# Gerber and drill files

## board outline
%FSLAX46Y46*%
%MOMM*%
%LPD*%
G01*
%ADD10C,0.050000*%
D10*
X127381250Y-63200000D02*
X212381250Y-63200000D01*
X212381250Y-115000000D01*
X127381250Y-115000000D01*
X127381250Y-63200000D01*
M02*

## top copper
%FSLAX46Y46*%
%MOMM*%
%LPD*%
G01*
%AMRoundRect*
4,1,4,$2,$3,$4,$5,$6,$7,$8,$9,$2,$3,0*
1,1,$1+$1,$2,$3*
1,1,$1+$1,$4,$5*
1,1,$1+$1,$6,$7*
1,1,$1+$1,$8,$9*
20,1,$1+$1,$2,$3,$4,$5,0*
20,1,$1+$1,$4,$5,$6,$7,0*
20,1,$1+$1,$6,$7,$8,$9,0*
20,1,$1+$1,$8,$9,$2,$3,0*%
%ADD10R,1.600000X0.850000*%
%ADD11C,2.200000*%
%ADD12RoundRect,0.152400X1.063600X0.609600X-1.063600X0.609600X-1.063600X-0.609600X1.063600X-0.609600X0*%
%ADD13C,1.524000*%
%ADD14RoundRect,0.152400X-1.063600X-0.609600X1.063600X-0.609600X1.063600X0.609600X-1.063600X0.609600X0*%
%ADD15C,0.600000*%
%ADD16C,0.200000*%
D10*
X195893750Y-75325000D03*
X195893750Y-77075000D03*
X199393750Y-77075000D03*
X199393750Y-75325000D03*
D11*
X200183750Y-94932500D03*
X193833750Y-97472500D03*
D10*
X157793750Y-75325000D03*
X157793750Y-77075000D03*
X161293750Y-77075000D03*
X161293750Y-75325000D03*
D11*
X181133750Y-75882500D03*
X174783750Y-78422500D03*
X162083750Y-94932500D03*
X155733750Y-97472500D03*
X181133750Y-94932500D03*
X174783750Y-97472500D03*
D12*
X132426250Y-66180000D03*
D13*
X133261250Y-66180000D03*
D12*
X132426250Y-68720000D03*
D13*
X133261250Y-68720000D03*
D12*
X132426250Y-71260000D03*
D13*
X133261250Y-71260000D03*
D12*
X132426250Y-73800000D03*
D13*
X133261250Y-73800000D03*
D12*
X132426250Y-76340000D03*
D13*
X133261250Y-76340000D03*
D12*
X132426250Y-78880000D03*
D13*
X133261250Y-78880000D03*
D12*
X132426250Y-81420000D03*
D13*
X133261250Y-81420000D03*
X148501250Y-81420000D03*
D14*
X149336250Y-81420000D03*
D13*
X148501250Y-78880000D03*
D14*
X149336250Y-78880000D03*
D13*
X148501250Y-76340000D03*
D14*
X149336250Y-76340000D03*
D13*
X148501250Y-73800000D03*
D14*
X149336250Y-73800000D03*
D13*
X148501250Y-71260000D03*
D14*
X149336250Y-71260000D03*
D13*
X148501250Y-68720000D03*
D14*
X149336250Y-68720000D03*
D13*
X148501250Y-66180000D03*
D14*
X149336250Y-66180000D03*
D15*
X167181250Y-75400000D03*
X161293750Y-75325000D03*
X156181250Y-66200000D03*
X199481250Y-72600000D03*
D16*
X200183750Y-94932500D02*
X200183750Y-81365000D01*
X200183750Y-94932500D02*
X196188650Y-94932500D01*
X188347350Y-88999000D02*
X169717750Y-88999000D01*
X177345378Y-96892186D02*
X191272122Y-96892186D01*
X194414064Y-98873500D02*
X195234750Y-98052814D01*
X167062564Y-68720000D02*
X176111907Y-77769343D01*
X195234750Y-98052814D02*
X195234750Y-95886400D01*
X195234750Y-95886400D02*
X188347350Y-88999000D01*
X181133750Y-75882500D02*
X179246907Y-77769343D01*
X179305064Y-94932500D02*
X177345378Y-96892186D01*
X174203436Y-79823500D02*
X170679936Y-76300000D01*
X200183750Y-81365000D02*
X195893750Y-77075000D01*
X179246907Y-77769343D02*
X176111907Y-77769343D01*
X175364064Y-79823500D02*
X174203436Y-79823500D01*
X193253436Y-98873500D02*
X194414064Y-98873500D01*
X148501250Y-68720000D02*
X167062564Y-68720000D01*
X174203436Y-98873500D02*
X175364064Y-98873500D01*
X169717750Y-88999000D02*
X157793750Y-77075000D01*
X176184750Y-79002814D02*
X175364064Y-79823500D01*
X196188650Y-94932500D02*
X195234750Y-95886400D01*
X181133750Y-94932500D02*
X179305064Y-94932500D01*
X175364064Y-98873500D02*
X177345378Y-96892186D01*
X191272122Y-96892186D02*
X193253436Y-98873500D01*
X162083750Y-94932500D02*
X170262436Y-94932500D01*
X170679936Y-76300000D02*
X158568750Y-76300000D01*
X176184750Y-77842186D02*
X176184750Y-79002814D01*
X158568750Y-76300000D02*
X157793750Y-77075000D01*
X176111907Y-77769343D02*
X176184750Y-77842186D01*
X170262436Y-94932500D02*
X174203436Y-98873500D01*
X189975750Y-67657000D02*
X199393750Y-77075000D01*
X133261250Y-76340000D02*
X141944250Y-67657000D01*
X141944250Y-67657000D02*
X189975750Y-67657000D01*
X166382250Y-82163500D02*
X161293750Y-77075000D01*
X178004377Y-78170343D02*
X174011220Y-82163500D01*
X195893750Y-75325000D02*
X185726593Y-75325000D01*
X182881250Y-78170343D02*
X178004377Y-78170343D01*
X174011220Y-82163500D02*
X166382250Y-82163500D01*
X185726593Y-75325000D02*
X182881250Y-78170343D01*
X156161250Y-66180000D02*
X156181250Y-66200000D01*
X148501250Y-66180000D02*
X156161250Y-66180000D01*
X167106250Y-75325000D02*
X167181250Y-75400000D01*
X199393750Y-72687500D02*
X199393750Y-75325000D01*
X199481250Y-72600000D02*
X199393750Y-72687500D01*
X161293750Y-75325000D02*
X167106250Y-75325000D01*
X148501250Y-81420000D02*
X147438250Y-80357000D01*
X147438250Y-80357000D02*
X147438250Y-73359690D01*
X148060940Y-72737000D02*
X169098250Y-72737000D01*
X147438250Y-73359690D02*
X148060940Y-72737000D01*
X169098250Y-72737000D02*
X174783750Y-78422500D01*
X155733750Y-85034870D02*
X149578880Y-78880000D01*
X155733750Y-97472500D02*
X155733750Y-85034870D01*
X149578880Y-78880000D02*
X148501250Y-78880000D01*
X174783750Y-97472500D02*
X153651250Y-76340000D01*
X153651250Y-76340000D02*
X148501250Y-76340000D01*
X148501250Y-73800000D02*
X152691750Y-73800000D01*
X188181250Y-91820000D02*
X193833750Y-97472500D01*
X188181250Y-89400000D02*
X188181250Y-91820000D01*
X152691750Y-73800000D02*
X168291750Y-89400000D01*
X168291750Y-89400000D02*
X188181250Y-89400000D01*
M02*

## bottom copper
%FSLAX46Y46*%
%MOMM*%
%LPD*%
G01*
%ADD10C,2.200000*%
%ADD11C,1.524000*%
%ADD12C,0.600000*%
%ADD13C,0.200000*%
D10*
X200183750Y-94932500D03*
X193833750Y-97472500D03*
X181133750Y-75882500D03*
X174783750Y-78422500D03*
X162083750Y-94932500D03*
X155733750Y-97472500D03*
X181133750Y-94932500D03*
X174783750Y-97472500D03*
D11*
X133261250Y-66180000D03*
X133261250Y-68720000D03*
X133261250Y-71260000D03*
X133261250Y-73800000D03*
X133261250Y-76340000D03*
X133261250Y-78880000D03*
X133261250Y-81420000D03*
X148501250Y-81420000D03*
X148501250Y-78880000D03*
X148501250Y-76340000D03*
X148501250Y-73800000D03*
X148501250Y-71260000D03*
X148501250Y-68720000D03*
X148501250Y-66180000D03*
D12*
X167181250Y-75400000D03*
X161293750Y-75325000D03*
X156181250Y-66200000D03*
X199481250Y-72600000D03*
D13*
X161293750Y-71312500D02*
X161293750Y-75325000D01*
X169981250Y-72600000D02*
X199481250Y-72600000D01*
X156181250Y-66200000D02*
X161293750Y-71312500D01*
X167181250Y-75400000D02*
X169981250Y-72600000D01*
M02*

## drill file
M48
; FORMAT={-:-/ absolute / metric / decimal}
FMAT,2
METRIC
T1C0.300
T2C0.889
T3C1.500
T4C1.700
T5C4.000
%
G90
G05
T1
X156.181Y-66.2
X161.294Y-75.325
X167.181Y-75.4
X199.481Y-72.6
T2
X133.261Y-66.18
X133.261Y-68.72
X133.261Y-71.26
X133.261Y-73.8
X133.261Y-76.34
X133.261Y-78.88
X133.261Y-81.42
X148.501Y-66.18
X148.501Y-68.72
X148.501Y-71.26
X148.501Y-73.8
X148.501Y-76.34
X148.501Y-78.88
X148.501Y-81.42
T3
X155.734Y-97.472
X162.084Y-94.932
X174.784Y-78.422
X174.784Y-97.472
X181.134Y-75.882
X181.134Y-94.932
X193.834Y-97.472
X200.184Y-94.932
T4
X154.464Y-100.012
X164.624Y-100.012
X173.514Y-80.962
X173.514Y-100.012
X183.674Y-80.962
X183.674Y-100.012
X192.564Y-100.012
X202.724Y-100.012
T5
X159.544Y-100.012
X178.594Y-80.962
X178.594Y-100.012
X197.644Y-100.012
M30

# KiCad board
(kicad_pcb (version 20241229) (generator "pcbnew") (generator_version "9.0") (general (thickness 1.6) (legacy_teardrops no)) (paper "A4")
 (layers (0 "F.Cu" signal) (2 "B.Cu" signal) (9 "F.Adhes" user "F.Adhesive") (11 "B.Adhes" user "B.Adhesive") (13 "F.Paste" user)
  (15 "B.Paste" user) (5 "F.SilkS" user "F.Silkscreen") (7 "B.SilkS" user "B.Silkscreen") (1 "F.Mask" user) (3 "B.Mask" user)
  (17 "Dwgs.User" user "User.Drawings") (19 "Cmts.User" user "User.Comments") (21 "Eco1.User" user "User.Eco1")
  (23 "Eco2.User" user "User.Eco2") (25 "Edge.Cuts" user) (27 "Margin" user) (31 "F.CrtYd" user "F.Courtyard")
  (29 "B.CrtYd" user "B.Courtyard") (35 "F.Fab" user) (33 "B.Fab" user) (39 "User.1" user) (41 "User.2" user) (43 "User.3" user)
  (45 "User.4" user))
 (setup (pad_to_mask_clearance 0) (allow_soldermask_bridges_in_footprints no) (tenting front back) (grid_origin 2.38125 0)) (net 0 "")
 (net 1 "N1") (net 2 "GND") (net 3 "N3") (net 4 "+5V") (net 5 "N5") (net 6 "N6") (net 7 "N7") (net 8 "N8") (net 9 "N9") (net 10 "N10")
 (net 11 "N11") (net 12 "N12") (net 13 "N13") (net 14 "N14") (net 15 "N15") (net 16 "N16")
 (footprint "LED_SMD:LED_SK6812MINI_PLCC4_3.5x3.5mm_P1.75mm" (layer "F.Cu") (at 197.64375 76.2)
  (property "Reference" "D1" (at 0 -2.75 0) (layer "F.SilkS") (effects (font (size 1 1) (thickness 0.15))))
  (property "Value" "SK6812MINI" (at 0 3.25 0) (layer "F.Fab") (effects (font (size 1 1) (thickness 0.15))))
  (pad "1" smd rect (at -1.75 -0.875) (size 1.6 0.85) (layers "F.Cu" "F.Mask" "F.Paste") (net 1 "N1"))
  (pad "2" smd rect (at -1.75 0.875) (size 1.6 0.85) (layers "F.Cu" "F.Mask" "F.Paste") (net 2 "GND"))
  (pad "3" smd rect (at 1.75 0.875) (size 1.6 0.85) (layers "F.Cu" "F.Mask" "F.Paste") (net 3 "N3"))
  (pad "4" smd rect (at 1.75 -0.875) (size 1.6 0.85) (layers "F.Cu" "F.Mask" "F.Paste") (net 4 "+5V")))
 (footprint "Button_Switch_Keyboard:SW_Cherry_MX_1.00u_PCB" (layer "F.Cu") (at 200.18375 94.9325)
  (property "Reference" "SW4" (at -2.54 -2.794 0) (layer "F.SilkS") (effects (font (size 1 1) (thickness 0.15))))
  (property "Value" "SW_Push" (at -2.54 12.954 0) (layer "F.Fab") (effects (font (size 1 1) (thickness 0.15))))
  (pad "" np_thru_hole circle (at -7.62 5.08) (size 1.7 1.7) (drill 1.7) (layers "*.Cu" "*.Mask"))
  (pad "" np_thru_hole circle (at -2.54 5.08) (size 4 4) (drill 4) (layers "*.Cu" "*.Mask"))
  (pad "" np_thru_hole circle (at 2.54 5.08) (size 1.7 1.7) (drill 1.7) (layers "*.Cu" "*.Mask"))
  (pad "1" thru_hole circle (at 0 0) (size 2.2 2.2) (drill 1.5) (layers "*.Cu" "*.Mask") (remove_unused_layers no) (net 2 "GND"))
  (pad "2" thru_hole circle (at -6.35 2.54) (size 2.2 2.2) (drill 1.5) (layers "*.Cu" "*.Mask") (remove_unused_layers no) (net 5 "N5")))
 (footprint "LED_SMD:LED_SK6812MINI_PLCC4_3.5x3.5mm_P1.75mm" (layer "F.Cu") (at 159.54375 76.2)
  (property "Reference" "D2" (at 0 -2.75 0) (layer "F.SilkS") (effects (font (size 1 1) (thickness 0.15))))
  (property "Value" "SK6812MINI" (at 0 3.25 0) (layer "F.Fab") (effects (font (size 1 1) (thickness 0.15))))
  (pad "1" smd rect (at -1.75 -0.875) (size 1.6 0.85) (layers "F.Cu" "F.Mask" "F.Paste") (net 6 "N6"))
  (pad "2" smd rect (at -1.75 0.875) (size 1.6 0.85) (layers "F.Cu" "F.Mask" "F.Paste") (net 2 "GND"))
  (pad "3" smd rect (at 1.75 0.875) (size 1.6 0.85) (layers "F.Cu" "F.Mask" "F.Paste") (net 1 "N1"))
  (pad "4" smd rect (at 1.75 -0.875) (size 1.6 0.85) (layers "F.Cu" "F.Mask" "F.Paste") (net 4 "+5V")))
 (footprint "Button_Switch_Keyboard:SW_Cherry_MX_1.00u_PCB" (layer "F.Cu") (at 181.13375 75.8825)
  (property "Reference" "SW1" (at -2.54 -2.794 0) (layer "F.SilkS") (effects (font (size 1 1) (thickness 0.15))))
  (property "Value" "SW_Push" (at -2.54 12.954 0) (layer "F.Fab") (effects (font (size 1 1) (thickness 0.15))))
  (pad "" np_thru_hole circle (at -7.62 5.08) (size 1.7 1.7) (drill 1.7) (layers "*.Cu" "*.Mask"))
  (pad "" np_thru_hole circle (at -2.54 5.08) (size 4 4) (drill 4) (layers "*.Cu" "*.Mask"))
  (pad "" np_thru_hole circle (at 2.54 5.08) (size 1.7 1.7) (drill 1.7) (layers "*.Cu" "*.Mask"))
  (pad "1" thru_hole circle (at 0 0) (size 2.2 2.2) (drill 1.5) (layers "*.Cu" "*.Mask") (remove_unused_layers no) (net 2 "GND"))
  (pad "2" thru_hole circle (at -6.35 2.54) (size 2.2 2.2) (drill 1.5) (layers "*.Cu" "*.Mask") (remove_unused_layers no) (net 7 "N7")))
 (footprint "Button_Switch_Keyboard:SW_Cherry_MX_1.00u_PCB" (layer "F.Cu") (at 162.08375 94.9325)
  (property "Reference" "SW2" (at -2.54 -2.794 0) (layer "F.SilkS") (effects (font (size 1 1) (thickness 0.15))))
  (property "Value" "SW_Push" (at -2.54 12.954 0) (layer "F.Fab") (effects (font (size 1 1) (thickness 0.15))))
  (pad "" np_thru_hole circle (at -7.62 5.08) (size 1.7 1.7) (drill 1.7) (layers "*.Cu" "*.Mask"))
  (pad "" np_thru_hole circle (at -2.54 5.08) (size 4 4) (drill 4) (layers "*.Cu" "*.Mask"))
  (pad "" np_thru_hole circle (at 2.54 5.08) (size 1.7 1.7) (drill 1.7) (layers "*.Cu" "*.Mask"))
  (pad "1" thru_hole circle (at 0 0) (size 2.2 2.2) (drill 1.5) (layers "*.Cu" "*.Mask") (remove_unused_layers no) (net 2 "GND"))
  (pad "2" thru_hole circle (at -6.35 2.54) (size 2.2 2.2) (drill 1.5) (layers "*.Cu" "*.Mask") (remove_unused_layers no) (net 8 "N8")))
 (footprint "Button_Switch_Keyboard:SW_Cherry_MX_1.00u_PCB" (layer "F.Cu") (at 181.13375 94.9325)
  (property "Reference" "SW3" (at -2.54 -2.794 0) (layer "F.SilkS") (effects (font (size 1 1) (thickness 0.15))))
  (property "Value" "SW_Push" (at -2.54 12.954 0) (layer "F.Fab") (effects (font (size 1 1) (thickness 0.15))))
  (pad "" np_thru_hole circle (at -7.62 5.08) (size 1.7 1.7) (drill 1.7) (layers "*.Cu" "*.Mask"))
  (pad "" np_thru_hole circle (at -2.54 5.08) (size 4 4) (drill 4) (layers "*.Cu" "*.Mask"))
  (pad "" np_thru_hole circle (at 2.54 5.08) (size 1.7 1.7) (drill 1.7) (layers "*.Cu" "*.Mask"))
  (pad "1" thru_hole circle (at 0 0) (size 2.2 2.2) (drill 1.5) (layers "*.Cu" "*.Mask") (remove_unused_layers no) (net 2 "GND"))
  (pad "2" thru_hole circle (at -6.35 2.54) (size 2.2 2.2) (drill 1.5) (layers "*.Cu" "*.Mask") (remove_unused_layers no) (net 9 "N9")))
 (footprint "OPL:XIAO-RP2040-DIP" (layer "F.Cu") (at 140.88125 73.8)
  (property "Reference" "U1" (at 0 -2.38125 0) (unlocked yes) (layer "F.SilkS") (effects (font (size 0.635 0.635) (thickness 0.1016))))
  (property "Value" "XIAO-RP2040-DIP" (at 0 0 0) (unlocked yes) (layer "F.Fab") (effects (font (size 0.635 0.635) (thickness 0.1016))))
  (pad "1" smd roundrect (at -8.455 -7.62 180) (size 2.432 1.524) (layers "F.Cu" "F.Mask") (roundrect_rratio 0.1) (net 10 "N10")
   (thermal_bridge_angle 45))
  (pad "1" thru_hole circle (at -7.62 -7.62 180) (size 1.524 1.524) (drill 0.889) (layers "*.Cu" "*.Mask") (remove_unused_layers no)
   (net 10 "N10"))
  (pad "2" smd roundrect (at -8.455 -5.08 180) (size 2.432 1.524) (layers "F.Cu" "F.Mask") (roundrect_rratio 0.1) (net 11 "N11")
   (thermal_bridge_angle 45))
  (pad "2" thru_hole circle (at -7.62 -5.08 180) (size 1.524 1.524) (drill 0.889) (layers "*.Cu" "*.Mask") (remove_unused_layers no)
   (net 11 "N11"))
  (pad "3" smd roundrect (at -8.455 -2.54 180) (size 2.432 1.524) (layers "F.Cu" "F.Mask") (roundrect_rratio 0.1) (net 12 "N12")
   (thermal_bridge_angle 45))
  (pad "3" thru_hole circle (at -7.62 -2.54 180) (size 1.524 1.524) (drill 0.889) (layers "*.Cu" "*.Mask") (remove_unused_layers no)
   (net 12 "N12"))
  (pad "4" smd roundrect (at -8.455 0 180) (size 2.432 1.524) (layers "F.Cu" "F.Mask") (roundrect_rratio 0.1) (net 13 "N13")
   (thermal_bridge_angle 45))
  (pad "4" thru_hole circle (at -7.62 0 180) (size 1.524 1.524) (drill 0.889) (layers "*.Cu" "*.Mask") (remove_unused_layers no)
   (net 13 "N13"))
  (pad "5" smd roundrect (at -8.455 2.54 180) (size 2.432 1.524) (layers "F.Cu" "F.Mask") (roundrect_rratio 0.1) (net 3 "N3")
   (thermal_bridge_angle 45))
  (pad "5" thru_hole circle (at -7.62 2.54 180) (size 1.524 1.524) (drill 0.889) (layers "*.Cu" "*.Mask") (remove_unused_layers no)
   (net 3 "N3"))
  (pad "6" smd roundrect (at -8.455 5.08 180) (size 2.432 1.524) (layers "F.Cu" "F.Mask") (roundrect_rratio 0.1) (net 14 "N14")
   (thermal_bridge_angle 45))
  (pad "6" thru_hole circle (at -7.62 5.08 180) (size 1.524 1.524) (drill 0.889) (layers "*.Cu" "*.Mask") (remove_unused_layers no)
   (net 14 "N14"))
  (pad "7" smd roundrect (at -8.455 7.62 180) (size 2.432 1.524) (layers "F.Cu" "F.Mask") (roundrect_rratio 0.1) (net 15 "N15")
   (thermal_bridge_angle 45))
  (pad "7" thru_hole circle (at -7.62 7.62 180) (size 1.524 1.524) (drill 0.889) (layers "*.Cu" "*.Mask") (remove_unused_layers no)
   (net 15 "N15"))
  (pad "8" thru_hole circle (at 7.62 7.62) (size 1.524 1.524) (drill 0.889) (layers "*.Cu" "*.Mask") (remove_unused_layers no) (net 7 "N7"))
  (pad "8" smd roundrect (at 8.455 7.62) (size 2.432 1.524) (layers "F.Cu" "F.Mask") (roundrect_rratio 0.1) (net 7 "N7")
   (thermal_bridge_angle 45))
  (pad "9" thru_hole circle (at 7.62 5.08) (size 1.524 1.524) (drill 0.889) (layers "*.Cu" "*.Mask") (remove_unused_layers no) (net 8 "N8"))
  (pad "9" smd roundrect (at 8.455 5.08) (size 2.432 1.524) (layers "F.Cu" "F.Mask") (roundrect_rratio 0.1) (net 8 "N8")
   (thermal_bridge_angle 45))
  (pad "10" thru_hole circle (at 7.62 2.54) (size 1.524 1.524) (drill 0.889) (layers "*.Cu" "*.Mask") (remove_unused_layers no) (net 9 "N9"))
  (pad "10" smd roundrect (at 8.455 2.54) (size 2.432 1.524) (layers "F.Cu" "F.Mask") (roundrect_rratio 0.1) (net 9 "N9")
   (thermal_bridge_angle 45))
  (pad "11" thru_hole circle (at 7.62 0) (size 1.524 1.524) (drill 0.889) (layers "*.Cu" "*.Mask") (remove_unused_layers no) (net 5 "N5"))
  (pad "11" smd roundrect (at 8.455 0) (size 2.432 1.524) (layers "F.Cu" "F.Mask") (roundrect_rratio 0.1) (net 5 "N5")
   (thermal_bridge_angle 45))
  (pad "12" thru_hole circle (at 7.62 -2.54) (size 1.524 1.524) (drill 0.889) (layers "*.Cu" "*.Mask") (remove_unused_layers no)
   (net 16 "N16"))
  (pad "12" smd roundrect (at 8.455 -2.54) (size 2.432 1.524) (layers "F.Cu" "F.Mask") (roundrect_rratio 0.1) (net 16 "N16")
   (thermal_bridge_angle 45))
  (pad "13" thru_hole circle (at 7.62 -5.08) (size 1.524 1.524) (drill 0.889) (layers "*.Cu" "*.Mask") (remove_unused_layers no)
   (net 2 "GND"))
  (pad "13" smd roundrect (at 8.455 -5.08) (size 2.432 1.524) (layers "F.Cu" "F.Mask") (roundrect_rratio 0.1) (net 2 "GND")
   (thermal_bridge_angle 45))
  (pad "14" thru_hole circle (at 7.62 -7.62) (size 1.524 1.524) (drill 0.889) (layers "*.Cu" "*.Mask") (remove_unused_layers no)
   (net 4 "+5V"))
  (pad "14" smd roundrect (at 8.455 -7.62) (size 2.432 1.524) (layers "F.Cu" "F.Mask") (roundrect_rratio 0.1) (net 4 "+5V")
   (thermal_bridge_angle 45)))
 (gr_rect (start 127.38125 63.2) (end 212.38125 115) (stroke (width 0.05) (type default)) (fill no) (layer "Edge.Cuts"))
 (segment (start 200.18375 94.9325) (end 200.18375 81.365) (width 0.2) (layer "F.Cu") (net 2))
 (segment (start 200.18375 94.9325) (end 196.18865 94.9325) (width 0.2) (layer "F.Cu") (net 2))
 (segment (start 188.34735 88.999) (end 169.71775 88.999) (width 0.2) (layer "F.Cu") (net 2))
 (segment (start 177.345378 96.892186) (end 191.272122 96.892186) (width 0.2) (layer "F.Cu") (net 2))
 (segment (start 194.414064 98.8735) (end 195.23475 98.052814) (width 0.2) (layer "F.Cu") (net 2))
 (segment (start 167.062564 68.72) (end 176.111907 77.769343) (width 0.2) (layer "F.Cu") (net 2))
 (segment (start 195.23475 98.052814) (end 195.23475 95.8864) (width 0.2) (layer "F.Cu") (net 2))
 (segment (start 195.23475 95.8864) (end 188.34735 88.999) (width 0.2) (layer "F.Cu") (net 2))
 (segment (start 181.13375 75.8825) (end 179.246907 77.769343) (width 0.2) (layer "F.Cu") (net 2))
 (segment (start 179.305064 94.9325) (end 177.345378 96.892186) (width 0.2) (layer "F.Cu") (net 2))
 (segment (start 174.203436 79.8235) (end 170.679936 76.3) (width 0.2) (layer "F.Cu") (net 2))
 (segment (start 200.18375 81.365) (end 195.89375 77.075) (width 0.2) (layer "F.Cu") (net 2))
 (segment (start 179.246907 77.769343) (end 176.111907 77.769343) (width 0.2) (layer "F.Cu") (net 2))
 (segment (start 175.364064 79.8235) (end 174.203436 79.8235) (width 0.2) (layer "F.Cu") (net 2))
 (segment (start 193.253436 98.8735) (end 194.414064 98.8735) (width 0.2) (layer "F.Cu") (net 2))
 (segment (start 148.50125 68.72) (end 167.062564 68.72) (width 0.2) (layer "F.Cu") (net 2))
 (segment (start 174.203436 98.8735) (end 175.364064 98.8735) (width 0.2) (layer "F.Cu") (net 2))
 (segment (start 169.71775 88.999) (end 157.79375 77.075) (width 0.2) (layer "F.Cu") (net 2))
 (segment (start 176.18475 79.002814) (end 175.364064 79.8235) (width 0.2) (layer "F.Cu") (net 2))
 (segment (start 196.18865 94.9325) (end 195.23475 95.8864) (width 0.2) (layer "F.Cu") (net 2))
 (segment (start 181.13375 94.9325) (end 179.305064 94.9325) (width 0.2) (layer "F.Cu") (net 2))
 (segment (start 175.364064 98.8735) (end 177.345378 96.892186) (width 0.2) (layer "F.Cu") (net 2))
 (segment (start 191.272122 96.892186) (end 193.253436 98.8735) (width 0.2) (layer "F.Cu") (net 2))
 (segment (start 162.08375 94.9325) (end 170.262436 94.9325) (width 0.2) (layer "F.Cu") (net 2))
 (segment (start 170.679936 76.3) (end 158.56875 76.3) (width 0.2) (layer "F.Cu") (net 2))
 (segment (start 176.18475 77.842186) (end 176.18475 79.002814) (width 0.2) (layer "F.Cu") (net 2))
 (segment (start 158.56875 76.3) (end 157.79375 77.075) (width 0.2) (layer "F.Cu") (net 2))
 (segment (start 176.111907 77.769343) (end 176.18475 77.842186) (width 0.2) (layer "F.Cu") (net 2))
 (segment (start 170.262436 94.9325) (end 174.203436 98.8735) (width 0.2) (layer "F.Cu") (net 2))
 (segment (start 189.97575 67.657) (end 199.39375 77.075) (width 0.2) (layer "F.Cu") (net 3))
 (segment (start 133.26125 76.34) (end 141.94425 67.657) (width 0.2) (layer "F.Cu") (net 3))
 (segment (start 141.94425 67.657) (end 189.97575 67.657) (width 0.2) (layer "F.Cu") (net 3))
 (segment (start 166.38225 82.1635) (end 161.29375 77.075) (width 0.2) (layer "F.Cu") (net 1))
 (segment (start 178.004377 78.170343) (end 174.01122 82.1635) (width 0.2) (layer "F.Cu") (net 1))
 (segment (start 195.89375 75.325) (end 185.726593 75.325) (width 0.2) (layer "F.Cu") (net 1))
 (segment (start 182.88125 78.170343) (end 178.004377 78.170343) (width 0.2) (layer "F.Cu") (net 1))
 (segment (start 174.01122 82.1635) (end 166.38225 82.1635) (width 0.2) (layer "F.Cu") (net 1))
 (segment (start 185.726593 75.325) (end 182.88125 78.170343) (width 0.2) (layer "F.Cu") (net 1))
 (segment (start 156.16125 66.18) (end 156.18125 66.2) (width 0.2) (layer "F.Cu") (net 4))
 (segment (start 148.50125 66.18) (end 156.16125 66.18) (width 0.2) (layer "F.Cu") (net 4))
 (segment (start 167.10625 75.325) (end 167.18125 75.4) (width 0.2) (layer "F.Cu") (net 4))
 (segment (start 199.39375 72.6875) (end 199.39375 75.325) (width 0.2) (layer "F.Cu") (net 4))
 (segment (start 199.48125 72.6) (end 199.39375 72.6875) (width 0.2) (layer "F.Cu") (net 4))
 (segment (start 161.29375 75.325) (end 167.10625 75.325) (width 0.2) (layer "F.Cu") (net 4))
 (via (at 167.18125 75.4) (size 0.6) (drill 0.3) (layers "F.Cu" "B.Cu") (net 4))
 (via (at 161.29375 75.325) (size 0.6) (drill 0.3) (layers "F.Cu" "B.Cu") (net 4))
 (via (at 156.18125 66.2) (size 0.6) (drill 0.3) (layers "F.Cu" "B.Cu") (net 4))
 (via (at 199.48125 72.6) (size 0.6) (drill 0.3) (layers "F.Cu" "B.Cu") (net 4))
 (segment (start 161.29375 71.3125) (end 161.29375 75.325) (width 0.2) (layer "B.Cu") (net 4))
 (segment (start 169.98125 72.6) (end 199.48125 72.6) (width 0.2) (layer "B.Cu") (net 4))
 (segment (start 156.18125 66.2) (end 161.29375 71.3125) (width 0.2) (layer "B.Cu") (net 4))
 (segment (start 167.18125 75.4) (end 169.98125 72.6) (width 0.2) (layer "B.Cu") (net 4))
 (segment (start 148.50125 81.42) (end 147.43825 80.357) (width 0.2) (layer "F.Cu") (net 7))
 (segment (start 147.43825 80.357) (end 147.43825 73.35969) (width 0.2) (layer "F.Cu") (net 7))
 (segment (start 148.06094 72.737) (end 169.09825 72.737) (width 0.2) (layer "F.Cu") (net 7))
 (segment (start 147.43825 73.35969) (end 148.06094 72.737) (width 0.2) (layer "F.Cu") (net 7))
 (segment (start 169.09825 72.737) (end 174.78375 78.4225) (width 0.2) (layer "F.Cu") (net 7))
 (segment (start 155.73375 85.03487) (end 149.57888 78.88) (width 0.2) (layer "F.Cu") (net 8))
 (segment (start 155.73375 97.4725) (end 155.73375 85.03487) (width 0.2) (layer "F.Cu") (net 8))
 (segment (start 149.57888 78.88) (end 148.50125 78.88) (width 0.2) (layer "F.Cu") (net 8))
 (segment (start 174.78375 97.4725) (end 153.65125 76.34) (width 0.2) (layer "F.Cu") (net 9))
 (segment (start 153.65125 76.34) (end 148.50125 76.34) (width 0.2) (layer "F.Cu") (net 9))
 (segment (start 148.50125 73.8) (end 152.69175 73.8) (width 0.2) (layer "F.Cu") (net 5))
 (segment (start 188.18125 91.82) (end 193.83375 97.4725) (width 0.2) (layer "F.Cu") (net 5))
 (segment (start 188.18125 89.4) (end 188.18125 91.82) (width 0.2) (layer "F.Cu") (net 5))
 (segment (start 152.69175 73.8) (end 168.29175 89.4) (width 0.2) (layer "F.Cu") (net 5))
 (segment (start 168.29175 89.4) (end 188.18125 89.4) (width 0.2) (layer "F.Cu") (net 5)))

